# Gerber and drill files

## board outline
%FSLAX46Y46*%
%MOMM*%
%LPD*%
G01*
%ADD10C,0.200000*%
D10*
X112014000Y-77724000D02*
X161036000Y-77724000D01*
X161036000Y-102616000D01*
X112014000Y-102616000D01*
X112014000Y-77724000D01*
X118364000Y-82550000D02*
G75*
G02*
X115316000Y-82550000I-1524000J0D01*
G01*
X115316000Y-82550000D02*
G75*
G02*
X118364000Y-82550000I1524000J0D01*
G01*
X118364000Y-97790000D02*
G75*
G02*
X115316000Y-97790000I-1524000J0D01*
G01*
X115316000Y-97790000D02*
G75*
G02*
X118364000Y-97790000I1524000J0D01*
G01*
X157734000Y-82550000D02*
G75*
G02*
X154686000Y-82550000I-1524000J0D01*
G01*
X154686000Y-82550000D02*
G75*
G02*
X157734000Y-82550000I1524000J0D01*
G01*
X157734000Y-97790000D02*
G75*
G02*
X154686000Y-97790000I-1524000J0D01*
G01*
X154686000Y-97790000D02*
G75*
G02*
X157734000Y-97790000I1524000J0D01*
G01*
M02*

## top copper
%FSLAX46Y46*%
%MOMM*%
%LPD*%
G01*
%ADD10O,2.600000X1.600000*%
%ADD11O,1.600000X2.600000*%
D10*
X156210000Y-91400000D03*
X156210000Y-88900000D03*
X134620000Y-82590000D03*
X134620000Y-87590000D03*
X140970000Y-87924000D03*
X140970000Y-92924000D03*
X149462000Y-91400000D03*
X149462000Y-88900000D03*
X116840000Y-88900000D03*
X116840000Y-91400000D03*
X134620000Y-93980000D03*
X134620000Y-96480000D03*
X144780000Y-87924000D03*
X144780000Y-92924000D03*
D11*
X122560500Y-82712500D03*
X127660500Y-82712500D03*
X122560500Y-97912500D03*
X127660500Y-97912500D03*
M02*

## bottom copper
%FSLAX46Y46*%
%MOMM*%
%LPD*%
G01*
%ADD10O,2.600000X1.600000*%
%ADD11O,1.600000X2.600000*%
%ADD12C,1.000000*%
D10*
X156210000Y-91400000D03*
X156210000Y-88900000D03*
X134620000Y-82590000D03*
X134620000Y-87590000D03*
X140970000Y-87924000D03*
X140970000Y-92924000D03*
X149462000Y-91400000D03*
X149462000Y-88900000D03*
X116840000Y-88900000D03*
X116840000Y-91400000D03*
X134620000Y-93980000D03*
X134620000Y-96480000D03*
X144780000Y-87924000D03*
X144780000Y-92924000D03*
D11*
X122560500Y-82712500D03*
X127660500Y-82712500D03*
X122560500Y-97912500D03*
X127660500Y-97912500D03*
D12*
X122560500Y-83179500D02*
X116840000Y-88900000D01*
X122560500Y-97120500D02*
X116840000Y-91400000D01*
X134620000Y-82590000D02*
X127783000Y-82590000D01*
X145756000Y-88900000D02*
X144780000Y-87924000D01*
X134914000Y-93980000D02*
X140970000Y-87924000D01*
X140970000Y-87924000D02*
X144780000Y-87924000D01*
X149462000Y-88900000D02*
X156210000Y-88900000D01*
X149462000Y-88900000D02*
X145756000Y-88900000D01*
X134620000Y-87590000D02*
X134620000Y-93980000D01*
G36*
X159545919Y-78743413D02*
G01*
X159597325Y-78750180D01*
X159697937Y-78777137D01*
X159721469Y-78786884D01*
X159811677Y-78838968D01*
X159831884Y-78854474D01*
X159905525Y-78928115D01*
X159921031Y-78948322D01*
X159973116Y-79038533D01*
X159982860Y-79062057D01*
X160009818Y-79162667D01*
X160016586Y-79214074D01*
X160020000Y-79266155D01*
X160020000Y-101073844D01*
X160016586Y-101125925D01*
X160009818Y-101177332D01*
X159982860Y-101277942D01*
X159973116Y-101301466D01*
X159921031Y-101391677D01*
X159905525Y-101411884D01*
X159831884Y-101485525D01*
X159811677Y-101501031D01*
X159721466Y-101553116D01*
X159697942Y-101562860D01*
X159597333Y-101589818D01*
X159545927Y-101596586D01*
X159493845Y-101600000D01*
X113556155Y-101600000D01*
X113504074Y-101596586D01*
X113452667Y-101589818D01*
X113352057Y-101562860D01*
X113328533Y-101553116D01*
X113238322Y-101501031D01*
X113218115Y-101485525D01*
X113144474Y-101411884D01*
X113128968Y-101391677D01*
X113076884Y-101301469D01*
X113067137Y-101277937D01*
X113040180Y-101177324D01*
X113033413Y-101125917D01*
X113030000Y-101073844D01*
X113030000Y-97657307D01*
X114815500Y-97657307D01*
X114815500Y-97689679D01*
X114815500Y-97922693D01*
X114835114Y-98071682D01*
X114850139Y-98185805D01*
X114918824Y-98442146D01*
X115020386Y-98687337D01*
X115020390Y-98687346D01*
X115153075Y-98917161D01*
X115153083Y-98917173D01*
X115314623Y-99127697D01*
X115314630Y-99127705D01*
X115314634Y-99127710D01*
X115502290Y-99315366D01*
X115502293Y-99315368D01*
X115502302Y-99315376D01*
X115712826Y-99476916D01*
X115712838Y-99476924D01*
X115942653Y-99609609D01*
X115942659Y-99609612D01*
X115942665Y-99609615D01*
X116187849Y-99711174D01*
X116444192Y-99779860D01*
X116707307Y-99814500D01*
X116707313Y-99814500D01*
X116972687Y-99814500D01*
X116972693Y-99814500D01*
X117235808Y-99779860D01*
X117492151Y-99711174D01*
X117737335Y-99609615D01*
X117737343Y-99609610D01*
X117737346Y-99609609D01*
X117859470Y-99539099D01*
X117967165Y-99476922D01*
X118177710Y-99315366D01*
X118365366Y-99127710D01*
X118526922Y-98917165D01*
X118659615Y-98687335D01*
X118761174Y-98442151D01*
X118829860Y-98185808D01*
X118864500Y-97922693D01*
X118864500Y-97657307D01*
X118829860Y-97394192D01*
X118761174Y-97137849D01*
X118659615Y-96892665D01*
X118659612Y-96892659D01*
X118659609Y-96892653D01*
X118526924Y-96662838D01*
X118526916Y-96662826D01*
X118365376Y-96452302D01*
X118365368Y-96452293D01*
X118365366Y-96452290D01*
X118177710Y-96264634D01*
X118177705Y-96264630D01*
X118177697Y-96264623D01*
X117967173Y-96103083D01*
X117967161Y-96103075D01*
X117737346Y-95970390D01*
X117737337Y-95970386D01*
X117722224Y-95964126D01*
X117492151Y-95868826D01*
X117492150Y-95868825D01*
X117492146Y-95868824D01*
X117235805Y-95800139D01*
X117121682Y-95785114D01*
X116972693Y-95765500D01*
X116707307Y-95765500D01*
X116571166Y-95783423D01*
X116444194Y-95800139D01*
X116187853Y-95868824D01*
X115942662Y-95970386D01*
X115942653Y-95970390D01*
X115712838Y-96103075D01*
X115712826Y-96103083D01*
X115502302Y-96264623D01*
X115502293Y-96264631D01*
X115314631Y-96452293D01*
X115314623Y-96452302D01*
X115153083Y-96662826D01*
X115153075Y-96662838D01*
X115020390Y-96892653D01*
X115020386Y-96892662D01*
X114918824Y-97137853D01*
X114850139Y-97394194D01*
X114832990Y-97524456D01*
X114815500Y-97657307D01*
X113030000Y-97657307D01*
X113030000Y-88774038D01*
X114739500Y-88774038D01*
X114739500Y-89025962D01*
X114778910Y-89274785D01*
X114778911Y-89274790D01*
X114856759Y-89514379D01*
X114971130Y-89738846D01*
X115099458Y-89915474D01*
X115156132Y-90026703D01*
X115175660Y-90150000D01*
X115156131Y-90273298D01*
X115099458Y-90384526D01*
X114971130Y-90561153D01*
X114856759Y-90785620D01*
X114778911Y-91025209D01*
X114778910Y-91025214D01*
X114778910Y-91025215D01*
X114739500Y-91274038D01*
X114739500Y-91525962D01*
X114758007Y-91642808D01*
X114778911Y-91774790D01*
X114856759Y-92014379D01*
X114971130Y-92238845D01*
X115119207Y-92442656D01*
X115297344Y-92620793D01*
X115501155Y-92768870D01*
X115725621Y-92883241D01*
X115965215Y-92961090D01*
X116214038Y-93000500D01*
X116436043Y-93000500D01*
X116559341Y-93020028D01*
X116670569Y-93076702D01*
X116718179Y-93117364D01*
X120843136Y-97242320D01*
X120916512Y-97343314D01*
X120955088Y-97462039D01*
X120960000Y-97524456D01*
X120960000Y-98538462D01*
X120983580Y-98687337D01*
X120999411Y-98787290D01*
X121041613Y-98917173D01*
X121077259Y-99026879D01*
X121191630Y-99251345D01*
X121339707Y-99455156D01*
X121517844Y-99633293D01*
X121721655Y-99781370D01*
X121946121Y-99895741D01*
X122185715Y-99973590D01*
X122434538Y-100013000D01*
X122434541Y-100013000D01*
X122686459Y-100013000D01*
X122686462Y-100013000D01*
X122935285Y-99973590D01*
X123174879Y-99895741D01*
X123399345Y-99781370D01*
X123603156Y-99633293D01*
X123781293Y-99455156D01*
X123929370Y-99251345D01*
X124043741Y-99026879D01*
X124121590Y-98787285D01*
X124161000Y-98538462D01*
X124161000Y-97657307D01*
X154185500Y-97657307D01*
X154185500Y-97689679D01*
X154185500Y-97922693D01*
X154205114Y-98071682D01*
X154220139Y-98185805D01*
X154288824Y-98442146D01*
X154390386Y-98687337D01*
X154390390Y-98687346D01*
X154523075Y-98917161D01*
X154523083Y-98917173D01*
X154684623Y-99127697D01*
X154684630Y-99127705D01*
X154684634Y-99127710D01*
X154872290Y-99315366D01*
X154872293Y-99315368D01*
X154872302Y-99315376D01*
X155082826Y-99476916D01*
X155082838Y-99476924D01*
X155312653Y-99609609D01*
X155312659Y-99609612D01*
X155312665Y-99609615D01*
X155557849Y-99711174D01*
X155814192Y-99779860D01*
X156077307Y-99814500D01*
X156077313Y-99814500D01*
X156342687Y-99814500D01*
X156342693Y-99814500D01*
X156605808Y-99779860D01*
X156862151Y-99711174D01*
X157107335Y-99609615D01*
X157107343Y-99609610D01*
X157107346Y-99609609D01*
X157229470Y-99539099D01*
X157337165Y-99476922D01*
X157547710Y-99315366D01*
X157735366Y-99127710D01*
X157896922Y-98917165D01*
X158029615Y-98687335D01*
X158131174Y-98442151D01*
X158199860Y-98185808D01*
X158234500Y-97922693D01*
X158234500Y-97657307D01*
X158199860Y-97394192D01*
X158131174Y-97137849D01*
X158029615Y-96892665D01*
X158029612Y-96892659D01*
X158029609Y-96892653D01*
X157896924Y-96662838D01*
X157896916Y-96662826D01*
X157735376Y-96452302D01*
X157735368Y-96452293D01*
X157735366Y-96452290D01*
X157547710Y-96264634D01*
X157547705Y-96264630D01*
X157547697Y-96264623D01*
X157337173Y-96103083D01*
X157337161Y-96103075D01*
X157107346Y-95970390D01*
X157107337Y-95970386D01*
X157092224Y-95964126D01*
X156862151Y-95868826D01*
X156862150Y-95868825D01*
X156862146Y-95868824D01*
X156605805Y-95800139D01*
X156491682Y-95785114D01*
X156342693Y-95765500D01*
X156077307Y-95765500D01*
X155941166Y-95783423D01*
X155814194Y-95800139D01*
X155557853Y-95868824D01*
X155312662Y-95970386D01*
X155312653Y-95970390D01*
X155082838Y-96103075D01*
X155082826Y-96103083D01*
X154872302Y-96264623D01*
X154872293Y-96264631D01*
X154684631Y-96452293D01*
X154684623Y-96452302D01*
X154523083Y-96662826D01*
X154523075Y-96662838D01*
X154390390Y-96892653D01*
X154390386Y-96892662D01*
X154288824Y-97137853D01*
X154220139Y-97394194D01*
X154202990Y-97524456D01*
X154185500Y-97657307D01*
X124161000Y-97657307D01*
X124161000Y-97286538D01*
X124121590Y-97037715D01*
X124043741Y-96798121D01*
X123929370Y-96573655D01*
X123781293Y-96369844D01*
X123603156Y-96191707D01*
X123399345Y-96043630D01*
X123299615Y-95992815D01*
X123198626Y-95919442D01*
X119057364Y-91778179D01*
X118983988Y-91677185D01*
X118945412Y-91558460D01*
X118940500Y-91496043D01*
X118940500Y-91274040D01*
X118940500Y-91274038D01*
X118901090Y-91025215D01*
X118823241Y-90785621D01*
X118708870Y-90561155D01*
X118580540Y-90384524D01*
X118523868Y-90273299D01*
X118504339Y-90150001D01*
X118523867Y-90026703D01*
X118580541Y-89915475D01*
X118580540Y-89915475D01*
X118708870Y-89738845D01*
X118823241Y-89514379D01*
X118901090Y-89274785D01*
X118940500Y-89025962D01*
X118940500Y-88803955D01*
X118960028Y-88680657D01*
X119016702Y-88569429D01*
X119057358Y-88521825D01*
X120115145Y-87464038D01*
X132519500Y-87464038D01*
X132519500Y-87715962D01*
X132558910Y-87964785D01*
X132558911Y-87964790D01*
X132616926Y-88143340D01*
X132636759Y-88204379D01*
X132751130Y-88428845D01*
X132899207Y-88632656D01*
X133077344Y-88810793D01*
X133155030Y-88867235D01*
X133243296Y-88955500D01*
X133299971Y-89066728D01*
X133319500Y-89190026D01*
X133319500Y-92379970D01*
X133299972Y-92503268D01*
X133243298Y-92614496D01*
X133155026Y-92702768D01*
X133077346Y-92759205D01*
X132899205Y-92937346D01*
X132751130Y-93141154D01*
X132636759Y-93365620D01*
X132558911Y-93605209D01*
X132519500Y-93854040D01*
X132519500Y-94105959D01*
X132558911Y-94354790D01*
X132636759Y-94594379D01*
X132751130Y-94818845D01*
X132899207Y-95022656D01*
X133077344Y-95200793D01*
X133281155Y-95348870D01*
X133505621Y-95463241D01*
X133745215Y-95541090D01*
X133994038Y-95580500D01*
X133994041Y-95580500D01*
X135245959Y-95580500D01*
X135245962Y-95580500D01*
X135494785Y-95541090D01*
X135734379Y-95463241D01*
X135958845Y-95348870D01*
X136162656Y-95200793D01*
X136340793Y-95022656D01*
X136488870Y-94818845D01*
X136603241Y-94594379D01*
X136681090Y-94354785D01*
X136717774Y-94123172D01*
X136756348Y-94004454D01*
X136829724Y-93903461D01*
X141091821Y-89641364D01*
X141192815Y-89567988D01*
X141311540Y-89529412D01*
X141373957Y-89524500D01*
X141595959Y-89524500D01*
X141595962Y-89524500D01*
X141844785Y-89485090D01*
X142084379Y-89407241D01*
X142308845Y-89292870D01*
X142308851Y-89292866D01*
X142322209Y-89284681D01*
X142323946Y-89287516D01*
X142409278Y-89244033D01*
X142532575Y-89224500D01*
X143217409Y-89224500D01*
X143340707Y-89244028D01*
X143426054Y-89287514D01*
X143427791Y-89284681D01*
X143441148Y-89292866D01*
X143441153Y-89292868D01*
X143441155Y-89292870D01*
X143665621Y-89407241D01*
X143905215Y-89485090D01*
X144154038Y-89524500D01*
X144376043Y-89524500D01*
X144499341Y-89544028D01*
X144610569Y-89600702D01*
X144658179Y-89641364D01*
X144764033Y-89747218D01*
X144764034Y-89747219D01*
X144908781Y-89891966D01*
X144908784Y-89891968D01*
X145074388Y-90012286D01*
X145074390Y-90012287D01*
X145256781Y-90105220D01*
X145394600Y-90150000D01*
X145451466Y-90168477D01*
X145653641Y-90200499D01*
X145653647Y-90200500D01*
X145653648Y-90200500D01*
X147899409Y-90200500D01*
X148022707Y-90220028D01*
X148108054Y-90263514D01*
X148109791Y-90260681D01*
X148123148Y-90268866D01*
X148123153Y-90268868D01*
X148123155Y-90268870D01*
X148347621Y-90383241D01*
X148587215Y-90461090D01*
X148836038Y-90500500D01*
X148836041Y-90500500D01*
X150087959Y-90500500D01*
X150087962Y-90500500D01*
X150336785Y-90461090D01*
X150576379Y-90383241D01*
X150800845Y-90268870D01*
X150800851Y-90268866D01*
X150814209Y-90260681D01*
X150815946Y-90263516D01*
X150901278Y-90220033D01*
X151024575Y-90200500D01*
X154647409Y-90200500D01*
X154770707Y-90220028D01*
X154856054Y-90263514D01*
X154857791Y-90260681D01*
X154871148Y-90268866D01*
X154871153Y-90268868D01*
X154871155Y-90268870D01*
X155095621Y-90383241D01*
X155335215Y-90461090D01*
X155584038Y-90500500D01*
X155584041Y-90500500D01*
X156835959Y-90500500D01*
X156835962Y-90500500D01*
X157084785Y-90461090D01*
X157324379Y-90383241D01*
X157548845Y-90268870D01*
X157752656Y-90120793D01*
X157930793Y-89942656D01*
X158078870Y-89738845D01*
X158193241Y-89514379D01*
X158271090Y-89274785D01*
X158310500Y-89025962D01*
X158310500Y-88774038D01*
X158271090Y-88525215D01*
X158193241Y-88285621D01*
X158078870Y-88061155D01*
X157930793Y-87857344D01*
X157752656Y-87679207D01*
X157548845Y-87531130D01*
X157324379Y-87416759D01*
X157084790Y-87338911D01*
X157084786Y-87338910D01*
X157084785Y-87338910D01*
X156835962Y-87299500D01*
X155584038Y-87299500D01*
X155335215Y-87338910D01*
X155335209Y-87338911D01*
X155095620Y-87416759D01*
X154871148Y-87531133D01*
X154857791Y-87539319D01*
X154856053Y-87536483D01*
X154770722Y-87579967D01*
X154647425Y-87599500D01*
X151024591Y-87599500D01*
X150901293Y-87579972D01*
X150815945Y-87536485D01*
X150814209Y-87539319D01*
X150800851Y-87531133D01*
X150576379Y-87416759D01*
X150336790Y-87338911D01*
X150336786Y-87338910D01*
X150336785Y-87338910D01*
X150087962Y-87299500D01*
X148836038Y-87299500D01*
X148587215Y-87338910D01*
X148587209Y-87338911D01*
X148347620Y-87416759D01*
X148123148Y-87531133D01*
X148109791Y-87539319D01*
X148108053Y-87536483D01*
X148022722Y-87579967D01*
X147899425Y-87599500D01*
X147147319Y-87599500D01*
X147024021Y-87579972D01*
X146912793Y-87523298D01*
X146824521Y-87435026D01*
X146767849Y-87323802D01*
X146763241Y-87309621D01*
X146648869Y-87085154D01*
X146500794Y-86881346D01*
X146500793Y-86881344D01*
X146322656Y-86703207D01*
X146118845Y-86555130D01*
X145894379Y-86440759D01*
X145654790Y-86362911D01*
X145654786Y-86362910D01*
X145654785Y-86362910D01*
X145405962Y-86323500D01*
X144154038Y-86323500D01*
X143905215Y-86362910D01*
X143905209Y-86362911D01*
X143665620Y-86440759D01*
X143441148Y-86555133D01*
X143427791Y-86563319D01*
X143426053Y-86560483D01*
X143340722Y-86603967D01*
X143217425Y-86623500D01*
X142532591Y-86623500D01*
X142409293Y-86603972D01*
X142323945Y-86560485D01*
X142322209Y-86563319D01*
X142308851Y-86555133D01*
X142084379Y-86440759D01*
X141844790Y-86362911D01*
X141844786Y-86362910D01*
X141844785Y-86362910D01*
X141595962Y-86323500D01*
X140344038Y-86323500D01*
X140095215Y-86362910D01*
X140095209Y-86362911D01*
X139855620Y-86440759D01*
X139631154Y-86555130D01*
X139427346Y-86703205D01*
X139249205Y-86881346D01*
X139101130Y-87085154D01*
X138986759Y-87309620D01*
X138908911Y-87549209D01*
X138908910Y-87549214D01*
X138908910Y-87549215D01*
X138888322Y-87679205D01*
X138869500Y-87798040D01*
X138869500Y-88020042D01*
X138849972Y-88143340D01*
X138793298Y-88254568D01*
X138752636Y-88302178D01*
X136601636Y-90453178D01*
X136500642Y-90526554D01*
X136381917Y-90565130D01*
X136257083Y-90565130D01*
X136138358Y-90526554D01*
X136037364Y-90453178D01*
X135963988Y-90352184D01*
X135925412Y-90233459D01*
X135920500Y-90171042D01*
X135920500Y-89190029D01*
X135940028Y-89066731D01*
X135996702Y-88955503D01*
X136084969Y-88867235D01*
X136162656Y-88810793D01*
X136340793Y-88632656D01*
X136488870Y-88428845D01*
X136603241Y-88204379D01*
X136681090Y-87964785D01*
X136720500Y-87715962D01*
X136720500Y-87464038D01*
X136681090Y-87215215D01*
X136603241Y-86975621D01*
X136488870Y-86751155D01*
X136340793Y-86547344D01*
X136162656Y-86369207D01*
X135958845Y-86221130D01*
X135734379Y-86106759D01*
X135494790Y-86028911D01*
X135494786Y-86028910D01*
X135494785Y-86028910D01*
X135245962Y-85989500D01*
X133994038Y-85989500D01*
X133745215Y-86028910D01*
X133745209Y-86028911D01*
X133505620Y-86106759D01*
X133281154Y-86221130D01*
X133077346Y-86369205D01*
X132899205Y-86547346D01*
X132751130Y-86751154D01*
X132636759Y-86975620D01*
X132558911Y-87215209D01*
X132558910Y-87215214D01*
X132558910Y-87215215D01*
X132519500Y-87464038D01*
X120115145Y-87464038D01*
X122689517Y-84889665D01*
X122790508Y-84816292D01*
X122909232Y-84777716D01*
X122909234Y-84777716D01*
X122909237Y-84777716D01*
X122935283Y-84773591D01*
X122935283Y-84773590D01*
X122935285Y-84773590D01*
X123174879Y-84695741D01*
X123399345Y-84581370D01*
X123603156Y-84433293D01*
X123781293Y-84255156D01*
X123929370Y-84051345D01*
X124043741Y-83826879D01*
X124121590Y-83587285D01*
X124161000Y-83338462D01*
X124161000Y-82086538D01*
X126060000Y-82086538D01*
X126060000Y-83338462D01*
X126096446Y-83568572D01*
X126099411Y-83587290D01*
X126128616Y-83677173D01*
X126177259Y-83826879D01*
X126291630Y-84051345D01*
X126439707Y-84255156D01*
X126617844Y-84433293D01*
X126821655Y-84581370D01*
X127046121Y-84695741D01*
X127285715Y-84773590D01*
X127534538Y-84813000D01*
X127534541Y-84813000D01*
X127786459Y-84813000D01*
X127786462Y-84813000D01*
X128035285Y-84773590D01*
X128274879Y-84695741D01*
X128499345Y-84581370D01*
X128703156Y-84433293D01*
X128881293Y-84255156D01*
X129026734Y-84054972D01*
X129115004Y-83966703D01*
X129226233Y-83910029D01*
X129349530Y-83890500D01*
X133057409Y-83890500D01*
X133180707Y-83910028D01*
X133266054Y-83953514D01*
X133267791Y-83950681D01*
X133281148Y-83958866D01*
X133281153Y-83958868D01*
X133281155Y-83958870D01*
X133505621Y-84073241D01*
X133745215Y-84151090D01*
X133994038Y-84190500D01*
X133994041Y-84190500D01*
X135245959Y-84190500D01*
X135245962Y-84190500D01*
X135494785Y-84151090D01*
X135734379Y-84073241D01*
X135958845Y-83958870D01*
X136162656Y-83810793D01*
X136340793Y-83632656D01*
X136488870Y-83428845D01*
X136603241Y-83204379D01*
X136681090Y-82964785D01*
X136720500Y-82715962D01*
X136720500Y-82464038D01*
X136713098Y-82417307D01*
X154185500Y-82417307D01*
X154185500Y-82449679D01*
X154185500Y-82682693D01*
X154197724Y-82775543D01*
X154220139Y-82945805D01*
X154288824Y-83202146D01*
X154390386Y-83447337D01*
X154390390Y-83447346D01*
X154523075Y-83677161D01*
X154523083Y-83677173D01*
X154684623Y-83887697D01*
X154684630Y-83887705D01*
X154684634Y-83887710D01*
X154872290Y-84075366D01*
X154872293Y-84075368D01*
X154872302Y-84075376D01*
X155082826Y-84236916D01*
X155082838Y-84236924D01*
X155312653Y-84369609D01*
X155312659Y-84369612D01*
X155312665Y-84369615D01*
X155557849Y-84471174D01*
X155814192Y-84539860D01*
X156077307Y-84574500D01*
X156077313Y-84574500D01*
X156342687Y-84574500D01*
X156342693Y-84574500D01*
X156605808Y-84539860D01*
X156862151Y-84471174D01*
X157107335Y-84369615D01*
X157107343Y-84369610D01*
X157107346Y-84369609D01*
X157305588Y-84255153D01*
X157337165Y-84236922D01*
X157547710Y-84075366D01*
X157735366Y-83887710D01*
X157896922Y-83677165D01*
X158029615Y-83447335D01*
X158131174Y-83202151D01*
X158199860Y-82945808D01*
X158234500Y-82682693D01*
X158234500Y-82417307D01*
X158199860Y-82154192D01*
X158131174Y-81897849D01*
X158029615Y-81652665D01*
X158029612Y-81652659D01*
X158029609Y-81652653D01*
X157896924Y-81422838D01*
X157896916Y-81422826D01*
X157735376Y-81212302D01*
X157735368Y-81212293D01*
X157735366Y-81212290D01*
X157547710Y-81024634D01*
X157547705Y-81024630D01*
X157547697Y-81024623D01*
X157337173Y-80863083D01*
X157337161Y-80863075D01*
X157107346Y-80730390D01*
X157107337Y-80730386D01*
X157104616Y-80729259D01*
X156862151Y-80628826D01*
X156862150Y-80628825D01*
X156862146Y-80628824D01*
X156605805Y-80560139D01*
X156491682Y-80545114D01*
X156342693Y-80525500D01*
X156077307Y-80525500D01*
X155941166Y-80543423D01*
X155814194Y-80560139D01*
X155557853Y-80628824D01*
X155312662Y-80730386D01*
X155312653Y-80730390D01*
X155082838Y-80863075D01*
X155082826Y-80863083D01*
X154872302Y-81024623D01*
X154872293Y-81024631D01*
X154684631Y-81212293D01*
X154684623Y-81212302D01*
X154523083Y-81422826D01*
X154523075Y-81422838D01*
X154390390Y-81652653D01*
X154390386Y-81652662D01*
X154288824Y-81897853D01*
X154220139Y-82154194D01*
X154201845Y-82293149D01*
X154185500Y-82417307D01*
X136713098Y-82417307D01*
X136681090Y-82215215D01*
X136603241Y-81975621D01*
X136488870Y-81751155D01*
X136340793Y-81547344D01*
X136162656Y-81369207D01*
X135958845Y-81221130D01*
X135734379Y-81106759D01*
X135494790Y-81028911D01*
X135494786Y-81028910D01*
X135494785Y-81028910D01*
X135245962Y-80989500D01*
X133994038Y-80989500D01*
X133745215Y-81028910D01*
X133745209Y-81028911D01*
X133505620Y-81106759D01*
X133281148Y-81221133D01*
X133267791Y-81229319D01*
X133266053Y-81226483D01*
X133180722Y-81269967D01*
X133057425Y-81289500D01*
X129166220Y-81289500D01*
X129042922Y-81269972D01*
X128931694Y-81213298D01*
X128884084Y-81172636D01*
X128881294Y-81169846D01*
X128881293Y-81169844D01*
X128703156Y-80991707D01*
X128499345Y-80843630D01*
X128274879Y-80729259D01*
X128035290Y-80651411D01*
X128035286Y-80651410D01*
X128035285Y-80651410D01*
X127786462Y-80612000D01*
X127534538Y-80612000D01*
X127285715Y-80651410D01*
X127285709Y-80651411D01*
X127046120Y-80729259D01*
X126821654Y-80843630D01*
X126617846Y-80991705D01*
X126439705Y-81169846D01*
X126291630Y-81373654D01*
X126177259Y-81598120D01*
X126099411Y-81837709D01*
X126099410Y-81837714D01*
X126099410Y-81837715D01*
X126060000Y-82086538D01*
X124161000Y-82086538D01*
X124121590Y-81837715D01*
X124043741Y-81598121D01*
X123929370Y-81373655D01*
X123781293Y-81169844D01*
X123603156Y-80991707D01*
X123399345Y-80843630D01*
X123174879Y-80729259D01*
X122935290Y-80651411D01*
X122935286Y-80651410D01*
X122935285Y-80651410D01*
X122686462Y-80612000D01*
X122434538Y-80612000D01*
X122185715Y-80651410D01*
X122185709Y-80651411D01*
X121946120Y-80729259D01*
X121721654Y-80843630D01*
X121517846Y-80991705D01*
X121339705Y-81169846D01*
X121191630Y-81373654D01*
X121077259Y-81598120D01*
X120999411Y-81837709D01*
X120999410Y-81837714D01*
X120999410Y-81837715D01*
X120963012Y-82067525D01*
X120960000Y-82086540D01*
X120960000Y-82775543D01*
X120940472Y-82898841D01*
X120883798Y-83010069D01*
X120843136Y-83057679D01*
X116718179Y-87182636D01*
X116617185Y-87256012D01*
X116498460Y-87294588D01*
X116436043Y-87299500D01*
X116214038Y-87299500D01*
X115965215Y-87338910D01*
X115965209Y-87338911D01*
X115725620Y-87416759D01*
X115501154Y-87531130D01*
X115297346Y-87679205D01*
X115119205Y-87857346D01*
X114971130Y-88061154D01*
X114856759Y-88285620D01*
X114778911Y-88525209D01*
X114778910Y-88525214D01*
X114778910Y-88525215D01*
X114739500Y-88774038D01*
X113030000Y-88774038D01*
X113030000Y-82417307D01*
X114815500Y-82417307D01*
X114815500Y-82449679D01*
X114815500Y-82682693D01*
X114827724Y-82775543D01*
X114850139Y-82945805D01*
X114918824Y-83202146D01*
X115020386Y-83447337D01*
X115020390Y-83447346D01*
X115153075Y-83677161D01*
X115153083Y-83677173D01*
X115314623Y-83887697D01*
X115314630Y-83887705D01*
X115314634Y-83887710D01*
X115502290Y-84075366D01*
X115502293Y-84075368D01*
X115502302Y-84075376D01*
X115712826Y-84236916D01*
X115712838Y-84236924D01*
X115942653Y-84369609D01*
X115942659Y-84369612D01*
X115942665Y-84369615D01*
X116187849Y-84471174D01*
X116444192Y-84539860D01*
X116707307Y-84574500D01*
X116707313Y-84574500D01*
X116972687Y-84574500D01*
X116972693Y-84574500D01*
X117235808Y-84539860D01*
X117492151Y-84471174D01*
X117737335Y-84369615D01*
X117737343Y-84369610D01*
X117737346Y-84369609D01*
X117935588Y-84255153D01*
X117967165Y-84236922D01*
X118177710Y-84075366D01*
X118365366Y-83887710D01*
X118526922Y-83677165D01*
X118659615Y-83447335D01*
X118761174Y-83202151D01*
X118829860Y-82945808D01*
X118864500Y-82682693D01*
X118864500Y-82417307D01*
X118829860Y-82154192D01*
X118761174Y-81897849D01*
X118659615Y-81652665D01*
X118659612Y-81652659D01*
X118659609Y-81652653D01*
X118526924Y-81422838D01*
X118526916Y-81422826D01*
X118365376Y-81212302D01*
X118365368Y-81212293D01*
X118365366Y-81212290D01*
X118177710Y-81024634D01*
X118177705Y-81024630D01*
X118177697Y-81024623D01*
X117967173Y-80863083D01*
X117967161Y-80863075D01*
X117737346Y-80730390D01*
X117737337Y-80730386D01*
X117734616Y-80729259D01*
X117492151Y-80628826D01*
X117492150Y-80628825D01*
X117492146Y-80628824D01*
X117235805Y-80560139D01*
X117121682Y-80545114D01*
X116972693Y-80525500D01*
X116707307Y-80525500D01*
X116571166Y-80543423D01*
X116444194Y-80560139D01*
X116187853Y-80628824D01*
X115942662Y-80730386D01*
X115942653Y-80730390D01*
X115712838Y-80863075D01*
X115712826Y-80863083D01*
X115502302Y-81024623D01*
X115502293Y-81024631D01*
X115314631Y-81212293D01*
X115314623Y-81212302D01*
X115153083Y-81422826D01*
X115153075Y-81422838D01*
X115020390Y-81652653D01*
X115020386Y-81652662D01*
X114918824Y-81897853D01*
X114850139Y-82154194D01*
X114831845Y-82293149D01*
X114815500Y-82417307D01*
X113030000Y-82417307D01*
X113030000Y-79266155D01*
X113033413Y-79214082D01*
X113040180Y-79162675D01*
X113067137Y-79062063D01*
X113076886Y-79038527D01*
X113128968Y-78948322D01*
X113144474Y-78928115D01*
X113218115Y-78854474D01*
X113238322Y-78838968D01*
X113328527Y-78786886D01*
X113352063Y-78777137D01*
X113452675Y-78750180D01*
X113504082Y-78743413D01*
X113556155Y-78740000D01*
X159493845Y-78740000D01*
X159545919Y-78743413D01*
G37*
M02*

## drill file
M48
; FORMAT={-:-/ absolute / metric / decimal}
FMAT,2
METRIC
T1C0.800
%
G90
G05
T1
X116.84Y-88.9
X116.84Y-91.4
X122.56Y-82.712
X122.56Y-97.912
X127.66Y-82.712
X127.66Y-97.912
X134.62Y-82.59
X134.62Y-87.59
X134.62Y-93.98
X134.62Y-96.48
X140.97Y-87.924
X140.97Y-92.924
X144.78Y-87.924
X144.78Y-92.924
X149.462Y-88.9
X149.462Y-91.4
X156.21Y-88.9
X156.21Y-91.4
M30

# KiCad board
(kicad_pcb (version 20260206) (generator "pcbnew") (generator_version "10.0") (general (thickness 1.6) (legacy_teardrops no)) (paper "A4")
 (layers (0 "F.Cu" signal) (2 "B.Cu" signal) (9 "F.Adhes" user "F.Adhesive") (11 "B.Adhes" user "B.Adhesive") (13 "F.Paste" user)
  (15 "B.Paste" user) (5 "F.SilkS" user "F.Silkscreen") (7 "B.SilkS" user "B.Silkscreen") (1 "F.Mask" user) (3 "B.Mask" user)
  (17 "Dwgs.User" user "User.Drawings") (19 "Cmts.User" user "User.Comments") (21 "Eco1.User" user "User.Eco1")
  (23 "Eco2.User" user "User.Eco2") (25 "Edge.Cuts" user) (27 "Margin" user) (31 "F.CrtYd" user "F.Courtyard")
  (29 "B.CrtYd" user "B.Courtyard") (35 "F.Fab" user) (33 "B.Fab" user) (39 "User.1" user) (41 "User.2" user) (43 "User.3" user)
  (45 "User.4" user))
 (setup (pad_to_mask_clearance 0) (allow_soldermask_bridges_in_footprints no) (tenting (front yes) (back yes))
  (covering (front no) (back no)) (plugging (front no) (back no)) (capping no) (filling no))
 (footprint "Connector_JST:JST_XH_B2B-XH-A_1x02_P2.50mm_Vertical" (layer "F.Cu") (at 156.21 91.4 90)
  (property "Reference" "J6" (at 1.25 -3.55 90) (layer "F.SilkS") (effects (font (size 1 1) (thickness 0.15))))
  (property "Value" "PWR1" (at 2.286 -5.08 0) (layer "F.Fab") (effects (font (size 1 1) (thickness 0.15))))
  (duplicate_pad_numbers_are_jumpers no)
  (pad "1" thru_hole oval (at 0 0 90) (size 1.6 2.6) (drill 0.8) (layers "*.Cu" "*.Mask") (remove_unused_layers no) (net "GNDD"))
  (pad "2" thru_hole oval (at 2.5 0 90) (size 1.6 2.6) (drill 0.8) (layers "*.Cu" "*.Mask") (remove_unused_layers no)
   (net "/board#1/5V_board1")))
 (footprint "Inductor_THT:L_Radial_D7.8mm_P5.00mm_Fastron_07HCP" (layer "F.Cu") (at 134.62 82.59 -90)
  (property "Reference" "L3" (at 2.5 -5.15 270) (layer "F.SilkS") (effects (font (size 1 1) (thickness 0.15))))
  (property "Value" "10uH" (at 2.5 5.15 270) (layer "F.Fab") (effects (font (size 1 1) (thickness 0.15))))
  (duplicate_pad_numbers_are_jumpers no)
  (pad "1" thru_hole oval (at 0 0) (size 2.6 1.6) (drill 0.8) (layers "*.Cu" "*.Mask") (remove_unused_layers no) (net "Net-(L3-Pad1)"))
  (pad "2" thru_hole oval (at 5 0) (size 2.6 1.6) (drill 0.8) (layers "*.Cu" "*.Mask") (remove_unused_layers no) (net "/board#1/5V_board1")))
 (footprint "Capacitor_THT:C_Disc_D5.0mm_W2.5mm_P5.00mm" (layer "F.Cu") (at 140.97 87.924 -90)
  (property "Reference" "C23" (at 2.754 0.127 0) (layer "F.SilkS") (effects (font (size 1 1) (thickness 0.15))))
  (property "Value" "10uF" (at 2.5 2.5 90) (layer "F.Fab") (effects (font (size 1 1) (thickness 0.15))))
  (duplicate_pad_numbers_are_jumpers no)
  (pad "1" thru_hole oval (at 0 0) (size 2.6 1.6) (drill 0.8) (layers "*.Cu" "*.Mask") (remove_unused_layers no) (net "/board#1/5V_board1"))
  (pad "2" thru_hole oval (at 5 0) (size 2.6 1.6) (drill 0.8) (layers "*.Cu" "*.Mask") (remove_unused_layers no) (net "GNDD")))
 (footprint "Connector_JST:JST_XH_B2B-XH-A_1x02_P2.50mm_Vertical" (layer "F.Cu") (at 149.462 91.4 90)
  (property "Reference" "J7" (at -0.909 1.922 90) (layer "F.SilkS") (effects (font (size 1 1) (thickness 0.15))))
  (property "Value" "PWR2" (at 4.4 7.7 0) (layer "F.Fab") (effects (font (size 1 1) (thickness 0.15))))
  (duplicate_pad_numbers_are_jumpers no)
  (pad "1" thru_hole oval (at 0 0 90) (size 1.6 2.6) (drill 0.8) (layers "*.Cu" "*.Mask") (remove_unused_layers no) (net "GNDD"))
  (pad "2" thru_hole oval (at 2.5 0 90) (size 1.6 2.6) (drill 0.8) (layers "*.Cu" "*.Mask") (remove_unused_layers no)
   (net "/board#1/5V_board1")))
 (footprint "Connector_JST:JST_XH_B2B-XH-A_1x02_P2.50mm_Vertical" (layer "F.Cu") (at 116.84 88.9 -90)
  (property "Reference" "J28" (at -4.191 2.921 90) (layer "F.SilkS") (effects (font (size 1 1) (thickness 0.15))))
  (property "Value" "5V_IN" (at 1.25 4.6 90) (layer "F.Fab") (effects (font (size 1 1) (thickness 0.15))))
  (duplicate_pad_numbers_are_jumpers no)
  (pad "1" thru_hole oval (at 0 0) (size 2.6 1.6) (drill 0.8) (layers "*.Cu" "*.Mask") (remove_unused_layers no) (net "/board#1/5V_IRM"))
  (pad "2" thru_hole oval (at 2.5 0) (size 2.6 1.6) (drill 0.8) (layers "*.Cu" "*.Mask") (remove_unused_layers no) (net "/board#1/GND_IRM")))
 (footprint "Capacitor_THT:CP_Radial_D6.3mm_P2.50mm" (layer "F.Cu") (at 134.62 93.98 -90)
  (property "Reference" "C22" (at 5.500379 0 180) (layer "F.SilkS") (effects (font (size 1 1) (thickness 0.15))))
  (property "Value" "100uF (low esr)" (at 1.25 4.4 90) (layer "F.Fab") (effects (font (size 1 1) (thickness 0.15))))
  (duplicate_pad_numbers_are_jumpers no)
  (pad "1" thru_hole oval (at 0 0) (size 2.6 1.6) (drill 0.8) (layers "*.Cu" "*.Mask") (remove_unused_layers no) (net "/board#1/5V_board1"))
  (pad "2" thru_hole oval (at 2.5 0) (size 2.6 1.6) (drill 0.8) (layers "*.Cu" "*.Mask") (remove_unused_layers no) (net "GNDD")))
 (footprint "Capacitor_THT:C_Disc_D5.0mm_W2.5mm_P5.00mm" (layer "F.Cu") (at 144.78 87.924 -90)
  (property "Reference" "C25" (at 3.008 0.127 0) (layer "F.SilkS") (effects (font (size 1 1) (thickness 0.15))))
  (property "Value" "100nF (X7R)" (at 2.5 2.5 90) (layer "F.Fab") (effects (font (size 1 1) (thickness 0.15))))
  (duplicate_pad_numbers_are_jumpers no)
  (pad "1" thru_hole oval (at 0 0) (size 2.6 1.6) (drill 0.8) (layers "*.Cu" "*.Mask") (remove_unused_layers no) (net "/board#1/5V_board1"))
  (pad "2" thru_hole oval (at 5 0) (size 2.6 1.6) (drill 0.8) (layers "*.Cu" "*.Mask") (remove_unused_layers no) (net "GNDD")))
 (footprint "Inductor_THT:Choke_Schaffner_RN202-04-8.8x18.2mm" (layer "F.Cu") (at 122.5605 82.7125)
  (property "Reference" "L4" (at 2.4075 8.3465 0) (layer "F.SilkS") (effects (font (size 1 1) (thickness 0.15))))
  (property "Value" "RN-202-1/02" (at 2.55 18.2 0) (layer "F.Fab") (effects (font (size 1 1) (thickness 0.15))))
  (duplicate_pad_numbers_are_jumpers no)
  (pad "1" thru_hole oval (at 0 0 90) (size 2.6 1.6) (drill 0.8) (layers "*.Cu" "*.Mask") (remove_unused_layers no) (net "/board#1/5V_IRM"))
  (pad "2" thru_hole oval (at 5.1 0 90) (size 2.6 1.6) (drill 0.8) (layers "*.Cu" "*.Mask") (remove_unused_layers no) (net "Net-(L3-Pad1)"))
  (pad "3" thru_hole oval (at 0 15.2 90) (size 2.6 1.6) (drill 0.8) (layers "*.Cu" "*.Mask") (remove_unused_layers no)
   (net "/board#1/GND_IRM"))
  (pad "4" thru_hole oval (at 5.1 15.2 90) (size 2.6 1.6) (drill 0.8) (layers "*.Cu" "*.Mask") (remove_unused_layers no) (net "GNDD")))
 (gr_rect (start 112.014 77.724) (end 161.036 102.616) (stroke (width 0.2) (type solid)) (fill no) (layer "Edge.Cuts"))
 (gr_circle (center 116.84 82.55) (end 118.364 82.55) (stroke (width 0.2) (type solid)) (fill no) (layer "Edge.Cuts"))
 (gr_circle (center 116.84 97.79) (end 118.364 97.79) (stroke (width 0.2) (type solid)) (fill no) (layer "Edge.Cuts"))
 (gr_circle (center 156.21 82.55) (end 157.734 82.55) (stroke (width 0.2) (type solid)) (fill no) (layer "Edge.Cuts"))
 (gr_circle (center 156.21 97.79) (end 157.734 97.79) (stroke (width 0.2) (type solid)) (fill no) (layer "Edge.Cuts"))
 (segment (start 122.5605 83.1795) (end 116.84 88.9) (width 1) (layer "B.Cu") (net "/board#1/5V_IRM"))
 (segment (start 122.5605 97.1205) (end 116.84 91.4) (width 1) (layer "B.Cu") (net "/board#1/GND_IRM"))
 (segment (start 134.62 82.59) (end 127.783 82.59) (width 1) (layer "B.Cu") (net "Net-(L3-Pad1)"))
 (segment (start 145.756 88.9) (end 144.78 87.924) (width 1) (layer "B.Cu") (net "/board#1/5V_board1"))
 (segment (start 134.914 93.98) (end 140.97 87.924) (width 1) (layer "B.Cu") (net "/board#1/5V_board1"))
 (segment (start 140.97 87.924) (end 144.78 87.924) (width 1) (layer "B.Cu") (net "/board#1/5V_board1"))
 (segment (start 149.462 88.9) (end 156.21 88.9) (width 1) (layer "B.Cu") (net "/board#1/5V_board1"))
 (segment (start 149.462 88.9) (end 145.756 88.9) (width 1) (layer "B.Cu") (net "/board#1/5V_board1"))
 (segment (start 134.62 87.59) (end 134.62 93.98) (width 1) (layer "B.Cu") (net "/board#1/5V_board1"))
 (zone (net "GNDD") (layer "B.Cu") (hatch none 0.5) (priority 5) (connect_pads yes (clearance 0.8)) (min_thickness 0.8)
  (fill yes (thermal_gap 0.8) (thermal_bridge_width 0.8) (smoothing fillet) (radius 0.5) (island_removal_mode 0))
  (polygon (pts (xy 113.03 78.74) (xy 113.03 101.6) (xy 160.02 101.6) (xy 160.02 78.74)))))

